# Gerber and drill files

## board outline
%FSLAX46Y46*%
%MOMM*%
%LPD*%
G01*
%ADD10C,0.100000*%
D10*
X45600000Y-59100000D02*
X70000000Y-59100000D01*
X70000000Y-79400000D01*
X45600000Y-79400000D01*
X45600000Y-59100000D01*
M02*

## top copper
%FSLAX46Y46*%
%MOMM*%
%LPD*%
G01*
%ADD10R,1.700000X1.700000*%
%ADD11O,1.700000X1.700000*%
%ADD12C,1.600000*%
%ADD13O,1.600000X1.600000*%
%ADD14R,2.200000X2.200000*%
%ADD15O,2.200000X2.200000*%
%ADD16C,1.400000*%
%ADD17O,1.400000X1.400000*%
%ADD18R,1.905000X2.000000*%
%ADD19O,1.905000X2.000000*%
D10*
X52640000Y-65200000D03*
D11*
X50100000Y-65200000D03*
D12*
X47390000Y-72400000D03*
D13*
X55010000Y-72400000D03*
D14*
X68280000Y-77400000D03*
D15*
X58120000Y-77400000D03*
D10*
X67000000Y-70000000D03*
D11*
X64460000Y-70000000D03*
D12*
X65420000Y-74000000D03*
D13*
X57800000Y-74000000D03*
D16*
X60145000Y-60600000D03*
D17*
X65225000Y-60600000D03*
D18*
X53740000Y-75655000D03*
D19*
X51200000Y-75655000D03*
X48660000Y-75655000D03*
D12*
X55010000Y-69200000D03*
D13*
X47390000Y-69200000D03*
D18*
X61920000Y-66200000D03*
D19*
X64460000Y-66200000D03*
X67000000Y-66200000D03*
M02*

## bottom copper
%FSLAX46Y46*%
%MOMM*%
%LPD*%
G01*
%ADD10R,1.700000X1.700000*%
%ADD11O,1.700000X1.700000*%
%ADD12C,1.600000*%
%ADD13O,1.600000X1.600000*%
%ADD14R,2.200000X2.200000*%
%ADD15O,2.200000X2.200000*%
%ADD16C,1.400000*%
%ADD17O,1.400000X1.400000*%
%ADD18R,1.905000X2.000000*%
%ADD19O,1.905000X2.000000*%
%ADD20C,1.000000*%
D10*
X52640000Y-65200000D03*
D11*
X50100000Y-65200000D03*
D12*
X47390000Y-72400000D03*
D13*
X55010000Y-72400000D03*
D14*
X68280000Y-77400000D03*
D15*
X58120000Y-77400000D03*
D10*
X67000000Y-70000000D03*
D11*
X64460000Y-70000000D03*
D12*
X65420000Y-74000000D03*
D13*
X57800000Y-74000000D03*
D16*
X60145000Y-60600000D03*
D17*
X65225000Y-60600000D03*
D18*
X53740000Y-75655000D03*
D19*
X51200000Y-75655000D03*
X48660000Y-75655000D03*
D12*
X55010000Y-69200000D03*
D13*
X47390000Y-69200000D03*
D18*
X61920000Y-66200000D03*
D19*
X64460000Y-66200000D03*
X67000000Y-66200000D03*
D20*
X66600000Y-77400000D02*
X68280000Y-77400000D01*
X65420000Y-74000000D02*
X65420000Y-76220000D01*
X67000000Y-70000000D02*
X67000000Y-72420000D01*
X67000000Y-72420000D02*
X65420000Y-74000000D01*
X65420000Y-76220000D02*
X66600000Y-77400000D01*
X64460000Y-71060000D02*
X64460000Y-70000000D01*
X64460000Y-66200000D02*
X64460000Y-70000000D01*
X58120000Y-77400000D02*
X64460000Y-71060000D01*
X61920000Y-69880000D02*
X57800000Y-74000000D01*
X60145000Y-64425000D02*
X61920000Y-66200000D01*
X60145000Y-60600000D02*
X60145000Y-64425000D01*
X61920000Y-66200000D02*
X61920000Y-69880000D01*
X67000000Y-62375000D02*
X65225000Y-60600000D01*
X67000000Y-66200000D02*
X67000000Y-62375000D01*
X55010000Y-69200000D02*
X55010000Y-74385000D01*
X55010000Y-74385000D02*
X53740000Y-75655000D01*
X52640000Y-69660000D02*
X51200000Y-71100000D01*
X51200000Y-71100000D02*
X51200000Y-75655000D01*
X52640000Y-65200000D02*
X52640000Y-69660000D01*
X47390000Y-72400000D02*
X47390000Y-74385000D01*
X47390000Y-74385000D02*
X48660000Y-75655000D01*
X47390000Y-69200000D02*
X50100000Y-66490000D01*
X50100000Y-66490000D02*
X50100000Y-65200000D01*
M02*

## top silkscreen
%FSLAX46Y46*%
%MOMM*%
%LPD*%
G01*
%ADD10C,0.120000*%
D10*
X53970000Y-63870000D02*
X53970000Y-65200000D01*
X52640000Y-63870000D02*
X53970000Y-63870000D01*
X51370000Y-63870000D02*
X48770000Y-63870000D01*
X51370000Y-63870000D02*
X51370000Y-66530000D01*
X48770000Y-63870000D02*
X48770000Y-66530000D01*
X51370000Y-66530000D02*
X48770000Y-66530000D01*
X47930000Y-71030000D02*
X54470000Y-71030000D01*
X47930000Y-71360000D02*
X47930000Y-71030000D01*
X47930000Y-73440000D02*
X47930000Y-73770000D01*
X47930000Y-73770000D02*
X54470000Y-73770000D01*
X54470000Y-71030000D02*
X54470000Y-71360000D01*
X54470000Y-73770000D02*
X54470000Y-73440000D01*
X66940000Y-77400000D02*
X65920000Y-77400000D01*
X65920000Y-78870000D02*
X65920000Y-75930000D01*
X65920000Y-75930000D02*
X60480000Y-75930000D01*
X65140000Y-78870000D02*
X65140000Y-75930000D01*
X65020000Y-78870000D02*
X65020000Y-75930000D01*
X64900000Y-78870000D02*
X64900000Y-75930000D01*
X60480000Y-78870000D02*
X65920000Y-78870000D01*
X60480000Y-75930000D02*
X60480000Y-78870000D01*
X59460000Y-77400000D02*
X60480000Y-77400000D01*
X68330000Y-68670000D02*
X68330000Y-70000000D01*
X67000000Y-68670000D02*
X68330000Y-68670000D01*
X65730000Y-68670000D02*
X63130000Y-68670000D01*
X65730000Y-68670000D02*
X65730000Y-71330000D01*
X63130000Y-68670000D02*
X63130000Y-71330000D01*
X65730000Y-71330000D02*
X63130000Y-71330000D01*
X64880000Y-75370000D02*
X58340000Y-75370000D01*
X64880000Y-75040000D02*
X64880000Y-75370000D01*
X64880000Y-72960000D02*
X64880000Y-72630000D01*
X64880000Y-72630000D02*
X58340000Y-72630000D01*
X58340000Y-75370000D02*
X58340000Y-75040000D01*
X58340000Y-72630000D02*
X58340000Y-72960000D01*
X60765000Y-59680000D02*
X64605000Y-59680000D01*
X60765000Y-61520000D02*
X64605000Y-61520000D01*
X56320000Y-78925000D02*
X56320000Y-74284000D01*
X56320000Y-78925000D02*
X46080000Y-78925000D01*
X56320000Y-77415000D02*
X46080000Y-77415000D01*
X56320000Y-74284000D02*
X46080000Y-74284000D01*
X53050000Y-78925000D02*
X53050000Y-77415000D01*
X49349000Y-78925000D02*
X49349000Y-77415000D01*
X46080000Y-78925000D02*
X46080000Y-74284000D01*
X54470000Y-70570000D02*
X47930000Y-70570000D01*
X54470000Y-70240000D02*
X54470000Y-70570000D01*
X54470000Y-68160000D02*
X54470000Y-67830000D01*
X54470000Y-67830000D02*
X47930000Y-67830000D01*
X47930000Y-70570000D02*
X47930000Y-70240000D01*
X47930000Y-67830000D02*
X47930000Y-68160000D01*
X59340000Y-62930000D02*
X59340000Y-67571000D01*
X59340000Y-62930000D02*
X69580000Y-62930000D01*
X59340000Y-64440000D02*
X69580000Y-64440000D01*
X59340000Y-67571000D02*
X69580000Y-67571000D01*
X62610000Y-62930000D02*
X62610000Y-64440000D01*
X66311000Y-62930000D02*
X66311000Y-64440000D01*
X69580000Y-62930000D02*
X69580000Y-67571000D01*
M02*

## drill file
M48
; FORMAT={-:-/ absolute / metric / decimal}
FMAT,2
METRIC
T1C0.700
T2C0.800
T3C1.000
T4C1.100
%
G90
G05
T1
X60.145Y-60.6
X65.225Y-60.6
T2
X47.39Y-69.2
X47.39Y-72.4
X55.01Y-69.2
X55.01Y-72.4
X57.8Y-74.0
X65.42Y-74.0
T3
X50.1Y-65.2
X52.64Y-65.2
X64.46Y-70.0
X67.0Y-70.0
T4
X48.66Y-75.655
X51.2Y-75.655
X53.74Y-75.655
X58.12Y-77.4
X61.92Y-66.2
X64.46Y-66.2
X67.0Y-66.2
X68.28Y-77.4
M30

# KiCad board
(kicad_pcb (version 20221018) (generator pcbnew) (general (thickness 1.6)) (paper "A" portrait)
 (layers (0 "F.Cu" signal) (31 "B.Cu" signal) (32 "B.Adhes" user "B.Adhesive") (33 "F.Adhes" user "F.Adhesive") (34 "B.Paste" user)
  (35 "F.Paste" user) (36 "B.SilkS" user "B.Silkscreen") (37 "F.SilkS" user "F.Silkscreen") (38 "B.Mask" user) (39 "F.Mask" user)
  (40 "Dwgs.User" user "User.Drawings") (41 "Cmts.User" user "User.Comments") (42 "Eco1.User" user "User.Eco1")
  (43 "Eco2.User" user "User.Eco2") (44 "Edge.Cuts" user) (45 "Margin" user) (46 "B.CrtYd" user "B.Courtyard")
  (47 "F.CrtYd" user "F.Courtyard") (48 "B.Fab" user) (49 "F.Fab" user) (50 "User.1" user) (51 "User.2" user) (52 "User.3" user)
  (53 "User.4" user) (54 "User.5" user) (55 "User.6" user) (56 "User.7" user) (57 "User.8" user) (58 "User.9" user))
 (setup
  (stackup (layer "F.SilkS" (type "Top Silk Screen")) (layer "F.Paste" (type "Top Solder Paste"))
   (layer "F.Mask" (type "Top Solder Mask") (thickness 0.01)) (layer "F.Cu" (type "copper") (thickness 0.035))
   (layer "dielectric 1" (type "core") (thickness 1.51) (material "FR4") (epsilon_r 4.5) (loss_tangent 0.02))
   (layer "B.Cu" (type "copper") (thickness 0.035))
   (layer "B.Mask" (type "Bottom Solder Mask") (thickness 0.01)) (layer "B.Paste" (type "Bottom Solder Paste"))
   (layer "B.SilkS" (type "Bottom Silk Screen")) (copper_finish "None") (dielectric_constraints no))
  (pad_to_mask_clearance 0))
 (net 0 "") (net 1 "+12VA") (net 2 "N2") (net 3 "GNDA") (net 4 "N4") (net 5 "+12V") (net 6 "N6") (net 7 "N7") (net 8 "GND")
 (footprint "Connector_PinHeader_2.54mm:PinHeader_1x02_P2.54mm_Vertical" (layer "F.Cu") (at 52.64 65.2 -90)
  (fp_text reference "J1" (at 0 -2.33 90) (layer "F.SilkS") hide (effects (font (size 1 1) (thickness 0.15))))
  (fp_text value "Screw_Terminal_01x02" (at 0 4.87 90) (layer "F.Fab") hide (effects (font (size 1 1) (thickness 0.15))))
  (fp_line (start -1.33 -1.33) (end 0 -1.33) (stroke (width 0.12) (type solid)) (layer "F.SilkS"))
  (fp_line (start -1.33 0) (end -1.33 -1.33) (stroke (width 0.12) (type solid)) (layer "F.SilkS"))
  (fp_line (start -1.33 1.27) (end -1.33 3.87) (stroke (width 0.12) (type solid)) (layer "F.SilkS"))
  (fp_line (start -1.33 1.27) (end 1.33 1.27) (stroke (width 0.12) (type solid)) (layer "F.SilkS"))
  (fp_line (start -1.33 3.87) (end 1.33 3.87) (stroke (width 0.12) (type solid)) (layer "F.SilkS"))
  (fp_line (start 1.33 1.27) (end 1.33 3.87) (stroke (width 0.12) (type solid)) (layer "F.SilkS"))
  (pad "1" thru_hole rect (at 0 0 270) (size 1.7 1.7) (drill 1) (layers "*.Cu" "*.Mask") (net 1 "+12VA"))
  (pad "2" thru_hole oval (at 0 2.54 270) (size 1.7 1.7) (drill 1) (layers "*.Cu" "*.Mask") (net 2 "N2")))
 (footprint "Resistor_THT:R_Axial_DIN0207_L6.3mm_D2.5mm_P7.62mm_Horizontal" (layer "F.Cu") (at 47.39 72.4)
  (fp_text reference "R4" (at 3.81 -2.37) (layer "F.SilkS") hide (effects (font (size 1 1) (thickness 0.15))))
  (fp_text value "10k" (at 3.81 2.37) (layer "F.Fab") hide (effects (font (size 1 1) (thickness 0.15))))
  (fp_line (start 0.54 -1.37) (end 7.08 -1.37) (stroke (width 0.12) (type solid)) (layer "F.SilkS"))
  (fp_line (start 0.54 -1.04) (end 0.54 -1.37) (stroke (width 0.12) (type solid)) (layer "F.SilkS"))
  (fp_line (start 0.54 1.04) (end 0.54 1.37) (stroke (width 0.12) (type solid)) (layer "F.SilkS"))
  (fp_line (start 0.54 1.37) (end 7.08 1.37) (stroke (width 0.12) (type solid)) (layer "F.SilkS"))
  (fp_line (start 7.08 -1.37) (end 7.08 -1.04) (stroke (width 0.12) (type solid)) (layer "F.SilkS"))
  (fp_line (start 7.08 1.37) (end 7.08 1.04) (stroke (width 0.12) (type solid)) (layer "F.SilkS"))
  (pad "1" thru_hole circle (at 0 0) (size 1.6 1.6) (drill 0.8) (layers "*.Cu" "*.Mask") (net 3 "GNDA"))
  (pad "2" thru_hole oval (at 7.62 0) (size 1.6 1.6) (drill 0.8) (layers "*.Cu" "*.Mask") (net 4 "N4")))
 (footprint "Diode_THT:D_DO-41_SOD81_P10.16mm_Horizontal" (layer "F.Cu") (at 68.28 77.4 180)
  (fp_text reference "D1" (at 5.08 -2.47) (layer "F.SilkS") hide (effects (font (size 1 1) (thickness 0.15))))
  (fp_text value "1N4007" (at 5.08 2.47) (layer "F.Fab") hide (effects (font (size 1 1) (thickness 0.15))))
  (fp_line (start 1.34 0) (end 2.36 0) (stroke (width 0.12) (type solid)) (layer "F.SilkS"))
  (fp_line (start 2.36 -1.47) (end 2.36 1.47) (stroke (width 0.12) (type solid)) (layer "F.SilkS"))
  (fp_line (start 2.36 1.47) (end 7.8 1.47) (stroke (width 0.12) (type solid)) (layer "F.SilkS"))
  (fp_line (start 3.14 -1.47) (end 3.14 1.47) (stroke (width 0.12) (type solid)) (layer "F.SilkS"))
  (fp_line (start 3.26 -1.47) (end 3.26 1.47) (stroke (width 0.12) (type solid)) (layer "F.SilkS"))
  (fp_line (start 3.38 -1.47) (end 3.38 1.47) (stroke (width 0.12) (type solid)) (layer "F.SilkS"))
  (fp_line (start 7.8 -1.47) (end 2.36 -1.47) (stroke (width 0.12) (type solid)) (layer "F.SilkS"))
  (fp_line (start 7.8 1.47) (end 7.8 -1.47) (stroke (width 0.12) (type solid)) (layer "F.SilkS"))
  (fp_line (start 8.82 0) (end 7.8 0) (stroke (width 0.12) (type solid)) (layer "F.SilkS"))
  (pad "1" thru_hole rect (at 0 0 180) (size 2.2 2.2) (drill 1.1) (layers "*.Cu" "*.Mask") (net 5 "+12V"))
  (pad "2" thru_hole oval (at 10.16 0 180) (size 2.2 2.2) (drill 1.1) (layers "*.Cu" "*.Mask") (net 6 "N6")))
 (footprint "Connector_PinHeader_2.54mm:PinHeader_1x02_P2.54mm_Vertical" (layer "F.Cu") (at 67 70 -90)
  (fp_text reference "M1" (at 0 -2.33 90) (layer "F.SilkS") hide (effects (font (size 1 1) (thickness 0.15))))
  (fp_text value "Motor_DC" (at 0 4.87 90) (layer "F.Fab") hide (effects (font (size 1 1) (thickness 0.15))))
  (fp_line (start -1.33 -1.33) (end 0 -1.33) (stroke (width 0.12) (type solid)) (layer "F.SilkS"))
  (fp_line (start -1.33 0) (end -1.33 -1.33) (stroke (width 0.12) (type solid)) (layer "F.SilkS"))
  (fp_line (start -1.33 1.27) (end -1.33 3.87) (stroke (width 0.12) (type solid)) (layer "F.SilkS"))
  (fp_line (start -1.33 1.27) (end 1.33 1.27) (stroke (width 0.12) (type solid)) (layer "F.SilkS"))
  (fp_line (start -1.33 3.87) (end 1.33 3.87) (stroke (width 0.12) (type solid)) (layer "F.SilkS"))
  (fp_line (start 1.33 1.27) (end 1.33 3.87) (stroke (width 0.12) (type solid)) (layer "F.SilkS"))
  (pad "1" thru_hole rect (at 0 0 270) (size 1.7 1.7) (drill 1) (layers "*.Cu" "*.Mask") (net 5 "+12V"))
  (pad "2" thru_hole oval (at 0 2.54 270) (size 1.7 1.7) (drill 1) (layers "*.Cu" "*.Mask") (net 6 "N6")))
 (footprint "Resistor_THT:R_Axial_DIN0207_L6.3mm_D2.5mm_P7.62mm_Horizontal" (layer "F.Cu") (at 65.42 74 180)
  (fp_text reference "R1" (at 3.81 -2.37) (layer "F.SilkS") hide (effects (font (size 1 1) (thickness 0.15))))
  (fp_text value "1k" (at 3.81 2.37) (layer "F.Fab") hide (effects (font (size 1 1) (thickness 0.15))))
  (fp_line (start 0.54 -1.37) (end 7.08 -1.37) (stroke (width 0.12) (type solid)) (layer "F.SilkS"))
  (fp_line (start 0.54 -1.04) (end 0.54 -1.37) (stroke (width 0.12) (type solid)) (layer "F.SilkS"))
  (fp_line (start 0.54 1.04) (end 0.54 1.37) (stroke (width 0.12) (type solid)) (layer "F.SilkS"))
  (fp_line (start 0.54 1.37) (end 7.08 1.37) (stroke (width 0.12) (type solid)) (layer "F.SilkS"))
  (fp_line (start 7.08 -1.37) (end 7.08 -1.04) (stroke (width 0.12) (type solid)) (layer "F.SilkS"))
  (fp_line (start 7.08 1.37) (end 7.08 1.04) (stroke (width 0.12) (type solid)) (layer "F.SilkS"))
  (pad "1" thru_hole circle (at 0 0 180) (size 1.6 1.6) (drill 0.8) (layers "*.Cu" "*.Mask") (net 5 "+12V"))
  (pad "2" thru_hole oval (at 7.62 0 180) (size 1.6 1.6) (drill 0.8) (layers "*.Cu" "*.Mask") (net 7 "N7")))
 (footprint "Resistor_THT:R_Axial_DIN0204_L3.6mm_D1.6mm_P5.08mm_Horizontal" (layer "F.Cu") (at 60.145 60.6)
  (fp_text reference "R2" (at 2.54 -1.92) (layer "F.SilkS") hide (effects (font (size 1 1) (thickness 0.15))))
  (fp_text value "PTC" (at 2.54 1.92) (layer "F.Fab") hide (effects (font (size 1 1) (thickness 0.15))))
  (fp_line (start 0.62 -0.92) (end 4.46 -0.92) (stroke (width 0.12) (type solid)) (layer "F.SilkS"))
  (fp_line (start 0.62 0.92) (end 4.46 0.92) (stroke (width 0.12) (type solid)) (layer "F.SilkS"))
  (pad "1" thru_hole circle (at 0 0) (size 1.4 1.4) (drill 0.7) (layers "*.Cu" "*.Mask") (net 7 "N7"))
  (pad "2" thru_hole oval (at 5.08 0) (size 1.4 1.4) (drill 0.7) (layers "*.Cu" "*.Mask") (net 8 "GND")))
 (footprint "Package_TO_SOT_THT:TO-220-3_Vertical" (layer "F.Cu") (at 53.74 75.655 180)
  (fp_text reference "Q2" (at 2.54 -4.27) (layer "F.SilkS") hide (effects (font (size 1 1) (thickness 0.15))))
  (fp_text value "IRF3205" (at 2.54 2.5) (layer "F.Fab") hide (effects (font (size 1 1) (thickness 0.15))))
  (fp_line (start -2.58 -3.27) (end -2.58 1.371) (stroke (width 0.12) (type solid)) (layer "F.SilkS"))
  (fp_line (start -2.58 -3.27) (end 7.66 -3.27) (stroke (width 0.12) (type solid)) (layer "F.SilkS"))
  (fp_line (start -2.58 -1.76) (end 7.66 -1.76) (stroke (width 0.12) (type solid)) (layer "F.SilkS"))
  (fp_line (start -2.58 1.371) (end 7.66 1.371) (stroke (width 0.12) (type solid)) (layer "F.SilkS"))
  (fp_line (start 0.69 -3.27) (end 0.69 -1.76) (stroke (width 0.12) (type solid)) (layer "F.SilkS"))
  (fp_line (start 4.391 -3.27) (end 4.391 -1.76) (stroke (width 0.12) (type solid)) (layer "F.SilkS"))
  (fp_line (start 7.66 -3.27) (end 7.66 1.371) (stroke (width 0.12) (type solid)) (layer "F.SilkS"))
  (pad "1" thru_hole rect (at 0 0 180) (size 1.905 2) (drill 1.1) (layers "*.Cu" "*.Mask") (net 4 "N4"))
  (pad "2" thru_hole oval (at 2.54 0 180) (size 1.905 2) (drill 1.1) (layers "*.Cu" "*.Mask") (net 1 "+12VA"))
  (pad "3" thru_hole oval (at 5.08 0 180) (size 1.905 2) (drill 1.1) (layers "*.Cu" "*.Mask") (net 3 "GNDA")))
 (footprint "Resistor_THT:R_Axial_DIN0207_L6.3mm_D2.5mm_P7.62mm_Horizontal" (layer "F.Cu") (at 55.01 69.2 180)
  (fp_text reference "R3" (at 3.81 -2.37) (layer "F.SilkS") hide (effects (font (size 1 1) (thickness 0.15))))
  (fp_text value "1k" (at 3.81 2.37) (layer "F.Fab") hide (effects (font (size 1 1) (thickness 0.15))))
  (fp_line (start 0.54 -1.37) (end 7.08 -1.37) (stroke (width 0.12) (type solid)) (layer "F.SilkS"))
  (fp_line (start 0.54 -1.04) (end 0.54 -1.37) (stroke (width 0.12) (type solid)) (layer "F.SilkS"))
  (fp_line (start 0.54 1.04) (end 0.54 1.37) (stroke (width 0.12) (type solid)) (layer "F.SilkS"))
  (fp_line (start 0.54 1.37) (end 7.08 1.37) (stroke (width 0.12) (type solid)) (layer "F.SilkS"))
  (fp_line (start 7.08 -1.37) (end 7.08 -1.04) (stroke (width 0.12) (type solid)) (layer "F.SilkS"))
  (fp_line (start 7.08 1.37) (end 7.08 1.04) (stroke (width 0.12) (type solid)) (layer "F.SilkS"))
  (pad "1" thru_hole circle (at 0 0 180) (size 1.6 1.6) (drill 0.8) (layers "*.Cu" "*.Mask") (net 4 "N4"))
  (pad "2" thru_hole oval (at 7.62 0 180) (size 1.6 1.6) (drill 0.8) (layers "*.Cu" "*.Mask") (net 2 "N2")))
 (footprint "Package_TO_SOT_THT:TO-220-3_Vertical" (layer "F.Cu") (at 61.92 66.2)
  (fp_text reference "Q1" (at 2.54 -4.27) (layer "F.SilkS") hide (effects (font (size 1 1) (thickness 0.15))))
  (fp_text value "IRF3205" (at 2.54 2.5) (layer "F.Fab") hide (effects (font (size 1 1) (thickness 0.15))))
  (fp_line (start -2.58 -3.27) (end -2.58 1.371) (stroke (width 0.12) (type solid)) (layer "F.SilkS"))
  (fp_line (start -2.58 -3.27) (end 7.66 -3.27) (stroke (width 0.12) (type solid)) (layer "F.SilkS"))
  (fp_line (start -2.58 -1.76) (end 7.66 -1.76) (stroke (width 0.12) (type solid)) (layer "F.SilkS"))
  (fp_line (start -2.58 1.371) (end 7.66 1.371) (stroke (width 0.12) (type solid)) (layer "F.SilkS"))
  (fp_line (start 0.69 -3.27) (end 0.69 -1.76) (stroke (width 0.12) (type solid)) (layer "F.SilkS"))
  (fp_line (start 4.391 -3.27) (end 4.391 -1.76) (stroke (width 0.12) (type solid)) (layer "F.SilkS"))
  (fp_line (start 7.66 -3.27) (end 7.66 1.371) (stroke (width 0.12) (type solid)) (layer "F.SilkS"))
  (pad "1" thru_hole rect (at 0 0) (size 1.905 2) (drill 1.1) (layers "*.Cu" "*.Mask") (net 7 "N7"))
  (pad "2" thru_hole oval (at 2.54 0) (size 1.905 2) (drill 1.1) (layers "*.Cu" "*.Mask") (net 6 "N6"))
  (pad "3" thru_hole oval (at 5.08 0) (size 1.905 2) (drill 1.1) (layers "*.Cu" "*.Mask") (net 8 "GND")))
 (gr_rect (start 45.6 59.1) (end 70 79.4) (stroke (width 0.1) (type default)) (fill none) (layer "Edge.Cuts"))
 (segment (start 66.6 77.4) (end 68.28 77.4) (width 1) (layer "B.Cu") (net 5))
 (segment (start 65.42 74) (end 65.42 76.22) (width 1) (layer "B.Cu") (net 5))
 (segment (start 67 70) (end 67 72.42) (width 1) (layer "B.Cu") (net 5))
 (segment (start 67 72.42) (end 65.42 74) (width 1) (layer "B.Cu") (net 5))
 (segment (start 65.42 76.22) (end 66.6 77.4) (width 1) (layer "B.Cu") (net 5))
 (segment (start 64.46 71.06) (end 64.46 70) (width 1) (layer "B.Cu") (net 6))
 (segment (start 64.46 66.2) (end 64.46 70) (width 1) (layer "B.Cu") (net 6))
 (segment (start 58.12 77.4) (end 64.46 71.06) (width 1) (layer "B.Cu") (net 6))
 (segment (start 61.92 69.88) (end 57.8 74) (width 1) (layer "B.Cu") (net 7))
 (segment (start 60.145 64.425) (end 61.92 66.2) (width 1) (layer "B.Cu") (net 7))
 (segment (start 60.145 60.6) (end 60.145 64.425) (width 1) (layer "B.Cu") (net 7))
 (segment (start 61.92 66.2) (end 61.92 69.88) (width 1) (layer "B.Cu") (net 7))
 (segment (start 67 62.375) (end 65.225 60.6) (width 1) (layer "B.Cu") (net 8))
 (segment (start 67 66.2) (end 67 62.375) (width 1) (layer "B.Cu") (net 8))
 (segment (start 55.01 69.2) (end 55.01 74.385) (width 1) (layer "B.Cu") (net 4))
 (segment (start 55.01 74.385) (end 53.74 75.655) (width 1) (layer "B.Cu") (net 4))
 (segment (start 52.64 69.66) (end 51.2 71.1) (width 1) (layer "B.Cu") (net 1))
 (segment (start 51.2 71.1) (end 51.2 75.655) (width 1) (layer "B.Cu") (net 1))
 (segment (start 52.64 65.2) (end 52.64 69.66) (width 1) (layer "B.Cu") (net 1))
 (segment (start 47.39 72.4) (end 47.39 74.385) (width 1) (layer "B.Cu") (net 3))
 (segment (start 47.39 74.385) (end 48.66 75.655) (width 1) (layer "B.Cu") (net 3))
 (segment (start 47.39 69.2) (end 50.1 66.49) (width 1) (layer "B.Cu") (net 2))
 (segment (start 50.1 66.49) (end 50.1 65.2) (width 1) (layer "B.Cu") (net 2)))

